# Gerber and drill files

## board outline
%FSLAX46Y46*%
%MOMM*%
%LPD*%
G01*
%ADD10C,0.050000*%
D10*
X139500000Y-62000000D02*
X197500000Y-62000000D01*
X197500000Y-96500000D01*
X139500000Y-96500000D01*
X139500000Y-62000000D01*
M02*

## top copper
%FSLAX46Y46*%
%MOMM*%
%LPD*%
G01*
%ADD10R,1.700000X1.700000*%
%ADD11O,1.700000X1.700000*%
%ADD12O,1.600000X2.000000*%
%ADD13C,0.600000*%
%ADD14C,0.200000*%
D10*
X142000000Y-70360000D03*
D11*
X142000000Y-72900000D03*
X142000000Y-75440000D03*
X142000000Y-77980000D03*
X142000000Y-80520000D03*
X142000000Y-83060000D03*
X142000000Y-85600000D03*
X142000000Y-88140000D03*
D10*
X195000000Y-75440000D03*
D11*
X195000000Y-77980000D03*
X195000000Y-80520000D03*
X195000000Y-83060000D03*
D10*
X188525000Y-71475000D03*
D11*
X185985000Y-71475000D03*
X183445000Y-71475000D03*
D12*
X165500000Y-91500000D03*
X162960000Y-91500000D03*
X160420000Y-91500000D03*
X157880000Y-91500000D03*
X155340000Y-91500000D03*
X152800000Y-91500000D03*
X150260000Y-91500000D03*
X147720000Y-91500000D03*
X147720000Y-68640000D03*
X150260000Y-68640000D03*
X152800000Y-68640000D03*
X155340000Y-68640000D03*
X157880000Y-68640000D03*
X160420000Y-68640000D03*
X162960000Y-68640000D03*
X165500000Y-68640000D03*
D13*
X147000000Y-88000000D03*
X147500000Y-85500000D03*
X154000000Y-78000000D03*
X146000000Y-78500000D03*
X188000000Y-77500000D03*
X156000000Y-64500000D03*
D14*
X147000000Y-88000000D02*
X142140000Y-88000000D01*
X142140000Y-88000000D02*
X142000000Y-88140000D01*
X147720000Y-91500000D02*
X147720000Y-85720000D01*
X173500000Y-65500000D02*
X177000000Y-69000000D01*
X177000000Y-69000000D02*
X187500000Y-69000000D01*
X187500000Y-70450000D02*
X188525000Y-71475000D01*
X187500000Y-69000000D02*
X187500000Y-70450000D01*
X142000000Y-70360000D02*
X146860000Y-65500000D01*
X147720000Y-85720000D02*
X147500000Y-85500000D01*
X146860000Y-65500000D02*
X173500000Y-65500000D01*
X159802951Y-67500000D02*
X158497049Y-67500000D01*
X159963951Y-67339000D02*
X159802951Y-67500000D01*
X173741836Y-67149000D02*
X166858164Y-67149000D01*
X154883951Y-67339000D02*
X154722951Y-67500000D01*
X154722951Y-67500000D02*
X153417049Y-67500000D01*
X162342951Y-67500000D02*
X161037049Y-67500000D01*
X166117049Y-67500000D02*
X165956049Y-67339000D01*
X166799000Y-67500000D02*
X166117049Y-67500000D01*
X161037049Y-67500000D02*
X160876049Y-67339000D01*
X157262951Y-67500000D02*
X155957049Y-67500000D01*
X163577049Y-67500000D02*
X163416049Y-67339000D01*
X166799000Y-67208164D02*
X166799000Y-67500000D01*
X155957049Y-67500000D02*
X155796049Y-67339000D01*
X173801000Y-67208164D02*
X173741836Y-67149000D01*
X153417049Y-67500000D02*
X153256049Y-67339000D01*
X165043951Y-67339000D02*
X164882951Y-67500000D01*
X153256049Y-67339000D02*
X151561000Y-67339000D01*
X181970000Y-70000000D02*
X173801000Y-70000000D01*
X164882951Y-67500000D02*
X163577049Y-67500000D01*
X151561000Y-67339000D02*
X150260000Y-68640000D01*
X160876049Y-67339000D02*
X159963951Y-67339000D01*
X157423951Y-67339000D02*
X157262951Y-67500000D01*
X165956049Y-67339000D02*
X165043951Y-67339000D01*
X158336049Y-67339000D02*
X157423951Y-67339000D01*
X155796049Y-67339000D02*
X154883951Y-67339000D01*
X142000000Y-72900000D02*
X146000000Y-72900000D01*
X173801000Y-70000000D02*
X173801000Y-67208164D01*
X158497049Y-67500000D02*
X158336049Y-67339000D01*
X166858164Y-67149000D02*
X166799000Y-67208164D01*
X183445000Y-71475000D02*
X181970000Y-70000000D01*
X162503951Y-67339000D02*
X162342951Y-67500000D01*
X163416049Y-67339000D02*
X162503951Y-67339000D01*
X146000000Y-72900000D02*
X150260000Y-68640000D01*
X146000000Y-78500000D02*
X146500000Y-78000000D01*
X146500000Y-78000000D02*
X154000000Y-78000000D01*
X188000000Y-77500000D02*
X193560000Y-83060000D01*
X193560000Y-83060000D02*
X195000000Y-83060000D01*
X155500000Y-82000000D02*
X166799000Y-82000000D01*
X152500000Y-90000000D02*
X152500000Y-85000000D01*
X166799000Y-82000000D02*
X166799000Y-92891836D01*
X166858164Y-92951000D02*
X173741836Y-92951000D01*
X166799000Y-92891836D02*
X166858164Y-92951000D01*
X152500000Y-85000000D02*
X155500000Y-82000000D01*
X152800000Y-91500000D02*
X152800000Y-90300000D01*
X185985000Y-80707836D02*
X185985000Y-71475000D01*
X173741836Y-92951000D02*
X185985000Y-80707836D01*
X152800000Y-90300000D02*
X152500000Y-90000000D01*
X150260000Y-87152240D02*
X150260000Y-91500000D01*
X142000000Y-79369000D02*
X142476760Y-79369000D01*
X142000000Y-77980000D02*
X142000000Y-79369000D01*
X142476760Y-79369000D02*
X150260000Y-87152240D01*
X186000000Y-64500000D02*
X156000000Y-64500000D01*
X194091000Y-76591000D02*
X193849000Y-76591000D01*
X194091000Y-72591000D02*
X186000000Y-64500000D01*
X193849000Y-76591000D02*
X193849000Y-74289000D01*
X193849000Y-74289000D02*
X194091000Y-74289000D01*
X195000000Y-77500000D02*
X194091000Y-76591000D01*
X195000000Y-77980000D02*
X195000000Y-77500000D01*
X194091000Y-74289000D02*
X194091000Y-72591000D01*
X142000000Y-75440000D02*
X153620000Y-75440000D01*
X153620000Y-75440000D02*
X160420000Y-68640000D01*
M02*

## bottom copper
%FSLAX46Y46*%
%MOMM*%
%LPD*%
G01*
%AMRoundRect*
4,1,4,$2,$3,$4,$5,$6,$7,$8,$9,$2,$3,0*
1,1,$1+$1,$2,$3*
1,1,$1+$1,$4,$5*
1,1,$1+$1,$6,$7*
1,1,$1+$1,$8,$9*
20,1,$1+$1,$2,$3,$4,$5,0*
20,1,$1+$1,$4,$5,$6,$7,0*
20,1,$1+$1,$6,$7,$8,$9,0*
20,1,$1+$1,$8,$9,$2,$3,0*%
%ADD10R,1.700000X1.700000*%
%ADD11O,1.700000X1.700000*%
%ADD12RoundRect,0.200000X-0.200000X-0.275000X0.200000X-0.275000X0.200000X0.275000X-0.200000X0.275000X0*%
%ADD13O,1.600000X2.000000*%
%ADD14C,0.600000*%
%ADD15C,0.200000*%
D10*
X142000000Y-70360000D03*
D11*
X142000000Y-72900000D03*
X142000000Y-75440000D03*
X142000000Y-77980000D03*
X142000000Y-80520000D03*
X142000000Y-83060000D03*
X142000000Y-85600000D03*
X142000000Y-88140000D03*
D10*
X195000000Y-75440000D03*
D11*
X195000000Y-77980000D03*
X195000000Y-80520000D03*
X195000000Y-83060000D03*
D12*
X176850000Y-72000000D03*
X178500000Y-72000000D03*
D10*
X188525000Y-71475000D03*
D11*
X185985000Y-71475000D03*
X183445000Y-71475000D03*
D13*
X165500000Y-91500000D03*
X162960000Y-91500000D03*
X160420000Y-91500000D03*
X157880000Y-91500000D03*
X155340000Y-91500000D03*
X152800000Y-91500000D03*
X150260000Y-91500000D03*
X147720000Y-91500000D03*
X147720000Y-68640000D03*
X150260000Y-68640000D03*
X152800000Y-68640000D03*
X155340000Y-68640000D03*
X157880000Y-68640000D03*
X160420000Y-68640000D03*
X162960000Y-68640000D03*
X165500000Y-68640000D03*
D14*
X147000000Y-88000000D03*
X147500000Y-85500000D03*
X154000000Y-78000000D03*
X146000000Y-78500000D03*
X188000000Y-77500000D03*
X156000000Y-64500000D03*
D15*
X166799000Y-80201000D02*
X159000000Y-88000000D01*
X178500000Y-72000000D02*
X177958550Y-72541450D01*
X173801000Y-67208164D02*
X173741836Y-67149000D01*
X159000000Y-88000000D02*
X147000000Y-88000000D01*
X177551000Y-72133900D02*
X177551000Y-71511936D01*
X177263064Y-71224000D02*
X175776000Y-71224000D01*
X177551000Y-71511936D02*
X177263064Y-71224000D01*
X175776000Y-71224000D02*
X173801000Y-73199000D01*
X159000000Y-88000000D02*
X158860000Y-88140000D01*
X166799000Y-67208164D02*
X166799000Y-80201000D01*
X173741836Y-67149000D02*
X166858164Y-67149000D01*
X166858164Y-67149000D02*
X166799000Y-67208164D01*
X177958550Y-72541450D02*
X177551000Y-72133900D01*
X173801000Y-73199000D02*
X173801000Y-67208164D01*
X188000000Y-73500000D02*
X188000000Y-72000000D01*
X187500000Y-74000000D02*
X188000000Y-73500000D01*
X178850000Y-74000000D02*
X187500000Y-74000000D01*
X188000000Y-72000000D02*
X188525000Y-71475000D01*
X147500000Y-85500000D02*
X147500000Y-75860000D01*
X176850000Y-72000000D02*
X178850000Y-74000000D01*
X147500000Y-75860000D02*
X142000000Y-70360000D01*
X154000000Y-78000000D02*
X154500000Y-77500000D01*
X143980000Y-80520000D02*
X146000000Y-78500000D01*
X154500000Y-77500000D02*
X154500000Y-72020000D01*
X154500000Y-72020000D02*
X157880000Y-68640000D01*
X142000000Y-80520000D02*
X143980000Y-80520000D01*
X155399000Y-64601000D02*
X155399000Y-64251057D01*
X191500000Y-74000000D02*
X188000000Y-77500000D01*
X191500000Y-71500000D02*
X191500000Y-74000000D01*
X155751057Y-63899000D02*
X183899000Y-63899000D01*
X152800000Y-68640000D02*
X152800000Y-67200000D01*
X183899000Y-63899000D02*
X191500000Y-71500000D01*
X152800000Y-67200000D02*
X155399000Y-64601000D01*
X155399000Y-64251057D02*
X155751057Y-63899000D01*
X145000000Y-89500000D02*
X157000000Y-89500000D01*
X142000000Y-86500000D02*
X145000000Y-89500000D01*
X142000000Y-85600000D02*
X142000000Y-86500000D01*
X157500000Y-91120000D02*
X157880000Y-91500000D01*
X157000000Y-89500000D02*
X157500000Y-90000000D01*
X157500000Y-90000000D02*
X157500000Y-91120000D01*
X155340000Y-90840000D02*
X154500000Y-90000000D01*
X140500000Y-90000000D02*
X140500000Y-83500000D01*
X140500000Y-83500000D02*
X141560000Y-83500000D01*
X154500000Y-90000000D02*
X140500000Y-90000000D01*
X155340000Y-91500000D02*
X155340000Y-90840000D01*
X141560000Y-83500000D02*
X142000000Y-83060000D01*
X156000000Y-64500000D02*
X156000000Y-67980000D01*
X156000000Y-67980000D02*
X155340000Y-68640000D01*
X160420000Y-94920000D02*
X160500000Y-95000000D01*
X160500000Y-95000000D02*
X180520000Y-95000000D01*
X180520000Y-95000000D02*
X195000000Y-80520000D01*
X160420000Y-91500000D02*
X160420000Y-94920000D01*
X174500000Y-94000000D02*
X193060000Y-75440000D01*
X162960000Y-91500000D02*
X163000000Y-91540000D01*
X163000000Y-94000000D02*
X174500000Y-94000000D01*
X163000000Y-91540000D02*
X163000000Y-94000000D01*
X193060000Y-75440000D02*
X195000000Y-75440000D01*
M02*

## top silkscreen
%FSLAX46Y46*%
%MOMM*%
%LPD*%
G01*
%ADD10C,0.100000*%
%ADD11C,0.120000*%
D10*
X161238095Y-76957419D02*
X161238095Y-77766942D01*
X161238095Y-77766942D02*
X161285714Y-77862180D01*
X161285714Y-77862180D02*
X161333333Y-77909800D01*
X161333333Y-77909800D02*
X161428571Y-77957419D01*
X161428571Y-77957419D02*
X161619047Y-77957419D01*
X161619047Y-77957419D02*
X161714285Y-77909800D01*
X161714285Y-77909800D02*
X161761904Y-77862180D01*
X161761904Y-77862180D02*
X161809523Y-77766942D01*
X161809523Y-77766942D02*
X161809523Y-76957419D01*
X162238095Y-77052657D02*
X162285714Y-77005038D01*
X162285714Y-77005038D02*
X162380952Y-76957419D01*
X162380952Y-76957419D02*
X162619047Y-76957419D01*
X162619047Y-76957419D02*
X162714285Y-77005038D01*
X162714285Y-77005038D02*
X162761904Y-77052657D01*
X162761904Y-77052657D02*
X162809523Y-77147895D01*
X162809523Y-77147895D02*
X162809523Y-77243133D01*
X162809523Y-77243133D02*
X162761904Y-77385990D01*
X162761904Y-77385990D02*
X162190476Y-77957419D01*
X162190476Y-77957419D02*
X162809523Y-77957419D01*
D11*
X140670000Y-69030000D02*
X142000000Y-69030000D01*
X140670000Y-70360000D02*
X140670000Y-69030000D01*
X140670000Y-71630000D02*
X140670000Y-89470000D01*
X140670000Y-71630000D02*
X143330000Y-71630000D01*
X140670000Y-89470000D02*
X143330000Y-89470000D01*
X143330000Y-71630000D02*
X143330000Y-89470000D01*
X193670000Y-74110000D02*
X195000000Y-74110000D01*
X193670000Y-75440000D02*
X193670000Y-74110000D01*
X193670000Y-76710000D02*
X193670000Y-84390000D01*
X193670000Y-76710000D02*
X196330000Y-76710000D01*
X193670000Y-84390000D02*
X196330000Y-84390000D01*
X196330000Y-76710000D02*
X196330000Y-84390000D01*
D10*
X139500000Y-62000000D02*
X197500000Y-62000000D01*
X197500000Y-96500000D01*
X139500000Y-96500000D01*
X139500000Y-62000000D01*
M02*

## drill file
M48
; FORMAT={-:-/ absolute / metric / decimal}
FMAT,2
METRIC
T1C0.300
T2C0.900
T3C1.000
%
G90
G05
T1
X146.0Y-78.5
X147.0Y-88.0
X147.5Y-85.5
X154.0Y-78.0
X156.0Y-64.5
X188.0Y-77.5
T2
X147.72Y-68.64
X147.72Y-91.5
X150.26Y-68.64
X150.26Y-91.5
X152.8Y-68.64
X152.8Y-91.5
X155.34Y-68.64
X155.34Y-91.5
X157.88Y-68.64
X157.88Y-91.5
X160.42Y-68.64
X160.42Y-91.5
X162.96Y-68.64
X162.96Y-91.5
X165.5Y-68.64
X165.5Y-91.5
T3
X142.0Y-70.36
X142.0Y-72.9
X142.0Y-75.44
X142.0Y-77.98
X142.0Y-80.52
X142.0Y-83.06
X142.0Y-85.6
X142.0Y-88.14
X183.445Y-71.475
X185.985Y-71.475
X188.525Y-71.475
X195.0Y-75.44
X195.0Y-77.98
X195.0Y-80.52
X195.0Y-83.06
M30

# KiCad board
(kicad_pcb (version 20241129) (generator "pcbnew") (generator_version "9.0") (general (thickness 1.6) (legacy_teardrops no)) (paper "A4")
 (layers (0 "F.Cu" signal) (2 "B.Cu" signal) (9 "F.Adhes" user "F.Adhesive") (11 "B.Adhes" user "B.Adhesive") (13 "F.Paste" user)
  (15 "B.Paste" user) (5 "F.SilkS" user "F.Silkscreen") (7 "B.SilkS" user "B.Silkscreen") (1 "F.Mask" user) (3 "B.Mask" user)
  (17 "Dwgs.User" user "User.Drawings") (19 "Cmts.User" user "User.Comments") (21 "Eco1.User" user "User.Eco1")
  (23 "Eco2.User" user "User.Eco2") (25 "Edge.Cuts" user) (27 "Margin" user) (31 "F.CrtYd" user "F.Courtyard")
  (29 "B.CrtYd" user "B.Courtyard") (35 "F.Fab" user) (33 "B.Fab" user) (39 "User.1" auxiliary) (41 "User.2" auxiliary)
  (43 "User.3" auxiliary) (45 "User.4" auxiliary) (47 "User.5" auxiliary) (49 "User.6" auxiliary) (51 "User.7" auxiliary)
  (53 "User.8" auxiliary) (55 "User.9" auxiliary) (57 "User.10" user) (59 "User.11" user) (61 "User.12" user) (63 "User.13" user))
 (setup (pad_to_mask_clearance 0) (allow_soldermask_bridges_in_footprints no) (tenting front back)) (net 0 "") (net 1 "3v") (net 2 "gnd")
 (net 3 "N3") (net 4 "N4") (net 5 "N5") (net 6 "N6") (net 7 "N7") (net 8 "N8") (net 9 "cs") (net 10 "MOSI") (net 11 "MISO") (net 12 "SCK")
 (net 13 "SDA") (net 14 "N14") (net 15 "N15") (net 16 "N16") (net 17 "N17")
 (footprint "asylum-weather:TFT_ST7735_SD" (layer "F.Cu") (at 162 79)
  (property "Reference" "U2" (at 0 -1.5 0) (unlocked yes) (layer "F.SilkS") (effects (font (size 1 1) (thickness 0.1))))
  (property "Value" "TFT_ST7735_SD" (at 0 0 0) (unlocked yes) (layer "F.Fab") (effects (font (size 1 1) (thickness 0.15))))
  (fp_line (start -21.33 -9.97) (end -20 -9.97) (stroke (width 0.12) (type solid)) (layer "F.SilkS"))
  (fp_line (start -21.33 -8.64) (end -21.33 -9.97) (stroke (width 0.12) (type solid)) (layer "F.SilkS"))
  (fp_line (start -21.33 -7.37) (end -21.33 10.47) (stroke (width 0.12) (type solid)) (layer "F.SilkS"))
  (fp_line (start -21.33 -7.37) (end -18.67 -7.37) (stroke (width 0.12) (type solid)) (layer "F.SilkS"))
  (fp_line (start -21.33 10.47) (end -18.67 10.47) (stroke (width 0.12) (type solid)) (layer "F.SilkS"))
  (fp_line (start -18.67 -7.37) (end -18.67 10.47) (stroke (width 0.12) (type solid)) (layer "F.SilkS"))
  (fp_line (start 31.67 -4.89) (end 33 -4.89) (stroke (width 0.12) (type solid)) (layer "F.SilkS"))
  (fp_line (start 31.67 -3.56) (end 31.67 -4.89) (stroke (width 0.12) (type solid)) (layer "F.SilkS"))
  (fp_line (start 31.67 -2.29) (end 31.67 5.39) (stroke (width 0.12) (type solid)) (layer "F.SilkS"))
  (fp_line (start 31.67 -2.29) (end 34.33 -2.29) (stroke (width 0.12) (type solid)) (layer "F.SilkS"))
  (fp_line (start 31.67 5.39) (end 34.33 5.39) (stroke (width 0.12) (type solid)) (layer "F.SilkS"))
  (fp_line (start 34.33 -2.29) (end 34.33 5.39) (stroke (width 0.12) (type solid)) (layer "F.SilkS"))
  (fp_rect (start -22.5 -17) (end 35.5 17.5) (stroke (width 0.1) (type default)) (fill no) (layer "F.SilkS"))
  (pad "1" thru_hole rect (at -20 -8.64) (size 1.7 1.7) (drill 1) (layers "*.Cu" "*.Mask") (remove_unused_layers no) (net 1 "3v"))
  (pad "2" thru_hole oval (at -20 -6.1) (size 1.7 1.7) (drill 1) (layers "*.Cu" "*.Mask") (remove_unused_layers no) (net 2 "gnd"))
  (pad "3" thru_hole oval (at -20 -3.56) (size 1.7 1.7) (drill 1) (layers "*.Cu" "*.Mask") (remove_unused_layers no) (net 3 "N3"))
  (pad "4" thru_hole oval (at -20 -1.02) (size 1.7 1.7) (drill 1) (layers "*.Cu" "*.Mask") (remove_unused_layers no) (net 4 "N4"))
  (pad "5" thru_hole oval (at -20 1.52) (size 1.7 1.7) (drill 1) (layers "*.Cu" "*.Mask") (remove_unused_layers no) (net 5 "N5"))
  (pad "6" thru_hole oval (at -20 4.06) (size 1.7 1.7) (drill 1) (layers "*.Cu" "*.Mask") (remove_unused_layers no) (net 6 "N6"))
  (pad "7" thru_hole oval (at -20 6.6) (size 1.7 1.7) (drill 1) (layers "*.Cu" "*.Mask") (remove_unused_layers no) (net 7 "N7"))
  (pad "8" thru_hole oval (at -20 9.14) (size 1.7 1.7) (drill 1) (layers "*.Cu" "*.Mask") (remove_unused_layers no) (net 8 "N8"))
  (pad "9" thru_hole rect (at 33 -3.56) (size 1.7 1.7) (drill 1) (layers "*.Cu" "*.Mask") (remove_unused_layers no) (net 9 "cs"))
  (pad "10" thru_hole oval (at 33 -1.02) (size 1.7 1.7) (drill 1) (layers "*.Cu" "*.Mask") (remove_unused_layers no) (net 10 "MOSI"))
  (pad "11" thru_hole oval (at 33 1.52) (size 1.7 1.7) (drill 1) (layers "*.Cu" "*.Mask") (remove_unused_layers no) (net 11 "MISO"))
  (pad "12" thru_hole oval (at 33 4.06) (size 1.7 1.7) (drill 1) (layers "*.Cu" "*.Mask") (remove_unused_layers no) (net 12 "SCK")))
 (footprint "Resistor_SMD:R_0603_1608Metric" (layer "B.Cu") (at 177.675 72)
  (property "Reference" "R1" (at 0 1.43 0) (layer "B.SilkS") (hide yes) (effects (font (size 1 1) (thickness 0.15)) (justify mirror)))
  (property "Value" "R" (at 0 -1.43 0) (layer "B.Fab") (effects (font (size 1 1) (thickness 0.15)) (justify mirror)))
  (pad "1" smd roundrect (at -0.825 0) (size 0.8 0.95) (layers "B.Cu" "B.Mask" "B.Paste") (roundrect_rratio 0.25) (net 1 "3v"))
  (pad "2" smd roundrect (at 0.825 0) (size 0.8 0.95) (layers "B.Cu" "B.Mask" "B.Paste") (roundrect_rratio 0.25) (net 8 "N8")))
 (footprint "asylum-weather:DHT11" (layer "B.Cu") (at 188.525 71.475 90)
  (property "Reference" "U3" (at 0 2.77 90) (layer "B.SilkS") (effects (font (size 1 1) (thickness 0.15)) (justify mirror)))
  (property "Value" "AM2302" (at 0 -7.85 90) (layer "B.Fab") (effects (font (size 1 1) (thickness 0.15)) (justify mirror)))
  (pad "1" thru_hole rect (at 0 0 90) (size 1.7 1.7) (drill 1) (layers "F&B.Cu" "*.Mask") (remove_unused_layers no) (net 1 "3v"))
  (pad "2" thru_hole oval (at 0 -2.54 90) (size 1.7 1.7) (drill 1) (layers "F&B.Cu" "*.Mask") (remove_unused_layers no) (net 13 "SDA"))
  (pad "3" thru_hole oval (at 0 -5.08 90) (size 1.7 1.7) (drill 1) (layers "F&B.Cu" "*.Mask") (remove_unused_layers no) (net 2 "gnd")))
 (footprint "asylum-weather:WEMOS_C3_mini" (layer "B.Cu") (at 158 80.07 90)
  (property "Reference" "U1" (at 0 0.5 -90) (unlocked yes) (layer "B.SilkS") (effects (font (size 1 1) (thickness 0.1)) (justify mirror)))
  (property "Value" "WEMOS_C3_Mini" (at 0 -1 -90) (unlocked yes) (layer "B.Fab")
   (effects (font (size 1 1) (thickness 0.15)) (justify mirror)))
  (pad "1" thru_hole oval (at -11.43 7.5 90) (size 2 1.6) (drill 0.9) (layers "F&B.Cu" "*.Mask") (remove_unused_layers no) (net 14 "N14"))
  (pad "2" thru_hole oval (at -11.43 4.96 90) (size 2 1.6) (drill 0.9) (layers "F&B.Cu" "*.Mask") (remove_unused_layers no) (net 9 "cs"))
  (pad "3" thru_hole oval (at -11.43 2.42 90) (size 2 1.6) (drill 0.9) (layers "F&B.Cu" "*.Mask") (remove_unused_layers no) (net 11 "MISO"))
  (pad "4" thru_hole oval (at -11.43 -0.12 90) (size 2 1.6) (drill 0.9) (layers "F&B.Cu" "*.Mask") (remove_unused_layers no) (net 7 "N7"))
  (pad "5" thru_hole oval (at -11.43 -2.66 90) (size 2 1.6) (drill 0.9) (layers "F&B.Cu" "*.Mask") (remove_unused_layers no) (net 6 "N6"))
  (pad "6" thru_hole oval (at -11.43 -5.2 90) (size 2 1.6) (drill 0.9) (layers "F&B.Cu" "*.Mask") (remove_unused_layers no) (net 13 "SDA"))
  (pad "7" thru_hole oval (at -11.43 -7.74 90) (size 2 1.6) (drill 0.9) (layers "F&B.Cu" "*.Mask") (remove_unused_layers no) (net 4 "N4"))
  (pad "8" thru_hole oval (at -11.43 -10.28 90) (size 2 1.6) (drill 0.9) (layers "F&B.Cu" "*.Mask") (remove_unused_layers no) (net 1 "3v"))
  (pad "9" thru_hole oval (at 11.43 -10.28 90) (size 2 1.6) (drill 0.9) (layers "F&B.Cu" "*.Mask") (remove_unused_layers no) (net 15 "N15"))
  (pad "10" thru_hole oval (at 11.43 -7.74 90) (size 2 1.6) (drill 0.9) (layers "F&B.Cu" "*.Mask") (remove_unused_layers no) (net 2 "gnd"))
  (pad "11" thru_hole oval (at 11.43 -5.2 90) (size 2 1.6) (drill 0.9) (layers "F&B.Cu" "*.Mask") (remove_unused_layers no) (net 12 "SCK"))
  (pad "12" thru_hole oval (at 11.43 -2.66 90) (size 2 1.6) (drill 0.9) (layers "F&B.Cu" "*.Mask") (remove_unused_layers no) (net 10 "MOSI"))
  (pad "13" thru_hole oval (at 11.43 -0.12 90) (size 2 1.6) (drill 0.9) (layers "F&B.Cu" "*.Mask") (remove_unused_layers no) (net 5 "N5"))
  (pad "14" thru_hole oval (at 11.43 2.42 90) (size 2 1.6) (drill 0.9) (layers "F&B.Cu" "*.Mask") (remove_unused_layers no) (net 3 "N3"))
  (pad "15" thru_hole oval (at 11.43 4.96 90) (size 2 1.6) (drill 0.9) (layers "F&B.Cu" "*.Mask") (remove_unused_layers no) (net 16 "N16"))
  (pad "16" thru_hole oval (at 11.43 7.5 90) (size 2 1.6) (drill 0.9) (layers "F&B.Cu" "*.Mask") (remove_unused_layers no) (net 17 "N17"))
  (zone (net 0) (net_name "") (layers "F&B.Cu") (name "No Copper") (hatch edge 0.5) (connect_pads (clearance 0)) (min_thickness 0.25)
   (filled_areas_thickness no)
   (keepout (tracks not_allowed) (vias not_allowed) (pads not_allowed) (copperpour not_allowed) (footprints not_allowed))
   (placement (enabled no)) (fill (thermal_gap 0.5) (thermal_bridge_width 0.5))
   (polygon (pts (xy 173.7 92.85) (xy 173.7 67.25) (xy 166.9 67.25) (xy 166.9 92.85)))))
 (gr_rect (start 139.5 62) (end 197.5 96.5) (stroke (width 0.05) (type default)) (fill no) (layer "Edge.Cuts"))
 (segment (start 147 88) (end 142.14 88) (width 0.2) (layer "F.Cu") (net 8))
 (segment (start 142.14 88) (end 142 88.14) (width 0.2) (layer "F.Cu") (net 8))
 (via (at 147 88) (size 0.6) (drill 0.3) (layers "F.Cu" "B.Cu") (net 8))
 (segment (start 166.799 80.201) (end 159 88) (width 0.2) (layer "B.Cu") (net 8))
 (segment (start 178.5 72) (end 177.95855 72.54145) (width 0.2) (layer "B.Cu") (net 8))
 (segment (start 173.801 67.208164) (end 173.741836 67.149) (width 0.2) (layer "B.Cu") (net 8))
 (segment (start 159 88) (end 147 88) (width 0.2) (layer "B.Cu") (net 8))
 (segment (start 177.551 72.1339) (end 177.551 71.511936) (width 0.2) (layer "B.Cu") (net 8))
 (segment (start 177.263064 71.224) (end 175.776 71.224) (width 0.2) (layer "B.Cu") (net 8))
 (segment (start 177.551 71.511936) (end 177.263064 71.224) (width 0.2) (layer "B.Cu") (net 8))
 (segment (start 175.776 71.224) (end 173.801 73.199) (width 0.2) (layer "B.Cu") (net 8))
 (segment (start 159 88) (end 158.86 88.14) (width 0.2) (layer "B.Cu") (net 8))
 (segment (start 166.799 67.208164) (end 166.799 80.201) (width 0.2) (layer "B.Cu") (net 8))
 (segment (start 173.741836 67.149) (end 166.858164 67.149) (width 0.2) (layer "B.Cu") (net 8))
 (segment (start 166.858164 67.149) (end 166.799 67.208164) (width 0.2) (layer "B.Cu") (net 8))
 (segment (start 177.95855 72.54145) (end 177.551 72.1339) (width 0.2) (layer "B.Cu") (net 8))
 (segment (start 173.801 73.199) (end 173.801 67.208164) (width 0.2) (layer "B.Cu") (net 8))
 (segment (start 147.72 91.5) (end 147.72 85.72) (width 0.2) (layer "F.Cu") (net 1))
 (segment (start 173.5 65.5) (end 177 69) (width 0.2) (layer "F.Cu") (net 1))
 (segment (start 177 69) (end 187.5 69) (width 0.2) (layer "F.Cu") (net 1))
 (segment (start 187.5 70.45) (end 188.525 71.475) (width 0.2) (layer "F.Cu") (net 1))
 (segment (start 187.5 69) (end 187.5 70.45) (width 0.2) (layer "F.Cu") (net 1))
 (segment (start 142 70.36) (end 146.86 65.5) (width 0.2) (layer "F.Cu") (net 1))
 (segment (start 147.72 85.72) (end 147.5 85.5) (width 0.2) (layer "F.Cu") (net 1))
 (segment (start 146.86 65.5) (end 173.5 65.5) (width 0.2) (layer "F.Cu") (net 1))
 (via (at 147.5 85.5) (size 0.6) (drill 0.3) (layers "F.Cu" "B.Cu") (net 1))
 (segment (start 188 73.5) (end 188 72) (width 0.2) (layer "B.Cu") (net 1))
 (segment (start 187.5 74) (end 188 73.5) (width 0.2) (layer "B.Cu") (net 1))
 (segment (start 178.85 74) (end 187.5 74) (width 0.2) (layer "B.Cu") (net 1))
 (segment (start 188 72) (end 188.525 71.475) (width 0.2) (layer "B.Cu") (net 1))
 (segment (start 147.5 85.5) (end 147.5 75.86) (width 0.2) (layer "B.Cu") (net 1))
 (segment (start 176.85 72) (end 178.85 74) (width 0.2) (layer "B.Cu") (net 1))
 (segment (start 147.5 75.86) (end 142 70.36) (width 0.2) (layer "B.Cu") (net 1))
 (segment (start 159.802951 67.5) (end 158.497049 67.5) (width 0.2) (layer "F.Cu") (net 2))
 (segment (start 159.963951 67.339) (end 159.802951 67.5) (width 0.2) (layer "F.Cu") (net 2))
 (segment (start 173.741836 67.149) (end 166.858164 67.149) (width 0.2) (layer "F.Cu") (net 2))
 (segment (start 154.883951 67.339) (end 154.722951 67.5) (width 0.2) (layer "F.Cu") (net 2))
 (segment (start 154.722951 67.5) (end 153.417049 67.5) (width 0.2) (layer "F.Cu") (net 2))
 (segment (start 162.342951 67.5) (end 161.037049 67.5) (width 0.2) (layer "F.Cu") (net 2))
 (segment (start 166.117049 67.5) (end 165.956049 67.339) (width 0.2) (layer "F.Cu") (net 2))
 (segment (start 166.799 67.5) (end 166.117049 67.5) (width 0.2) (layer "F.Cu") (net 2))
 (segment (start 161.037049 67.5) (end 160.876049 67.339) (width 0.2) (layer "F.Cu") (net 2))
 (segment (start 157.262951 67.5) (end 155.957049 67.5) (width 0.2) (layer "F.Cu") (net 2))
 (segment (start 163.577049 67.5) (end 163.416049 67.339) (width 0.2) (layer "F.Cu") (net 2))
 (segment (start 166.799 67.208164) (end 166.799 67.5) (width 0.2) (layer "F.Cu") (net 2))
 (segment (start 155.957049 67.5) (end 155.796049 67.339) (width 0.2) (layer "F.Cu") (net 2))
 (segment (start 173.801 67.208164) (end 173.741836 67.149) (width 0.2) (layer "F.Cu") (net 2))
 (segment (start 153.417049 67.5) (end 153.256049 67.339) (width 0.2) (layer "F.Cu") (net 2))
 (segment (start 165.043951 67.339) (end 164.882951 67.5) (width 0.2) (layer "F.Cu") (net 2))
 (segment (start 153.256049 67.339) (end 151.561 67.339) (width 0.2) (layer "F.Cu") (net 2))
 (segment (start 181.97 70) (end 173.801 70) (width 0.2) (layer "F.Cu") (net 2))
 (segment (start 164.882951 67.5) (end 163.577049 67.5) (width 0.2) (layer "F.Cu") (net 2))
 (segment (start 151.561 67.339) (end 150.26 68.64) (width 0.2) (layer "F.Cu") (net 2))
 (segment (start 160.876049 67.339) (end 159.963951 67.339) (width 0.2) (layer "F.Cu") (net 2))
 (segment (start 157.423951 67.339) (end 157.262951 67.5) (width 0.2) (layer "F.Cu") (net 2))
 (segment (start 165.956049 67.339) (end 165.043951 67.339) (width 0.2) (layer "F.Cu") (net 2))
 (segment (start 158.336049 67.339) (end 157.423951 67.339) (width 0.2) (layer "F.Cu") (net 2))
 (segment (start 155.796049 67.339) (end 154.883951 67.339) (width 0.2) (layer "F.Cu") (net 2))
 (segment (start 142 72.9) (end 146 72.9) (width 0.2) (layer "F.Cu") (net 2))
 (segment (start 173.801 70) (end 173.801 67.208164) (width 0.2) (layer "F.Cu") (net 2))
 (segment (start 158.497049 67.5) (end 158.336049 67.339) (width 0.2) (layer "F.Cu") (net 2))
 (segment (start 166.858164 67.149) (end 166.799 67.208164) (width 0.2) (layer "F.Cu") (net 2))
 (segment (start 183.445 71.475) (end 181.97 70) (width 0.2) (layer "F.Cu") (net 2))
 (segment (start 162.503951 67.339) (end 162.342951 67.5) (width 0.2) (layer "F.Cu") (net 2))
 (segment (start 163.416049 67.339) (end 162.503951 67.339) (width 0.2) (layer "F.Cu") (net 2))
 (segment (start 146 72.9) (end 150.26 68.64) (width 0.2) (layer "F.Cu") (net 2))
 (segment (start 146 78.5) (end 146.5 78) (width 0.2) (layer "F.Cu") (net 5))
 (segment (start 146.5 78) (end 154 78) (width 0.2) (layer "F.Cu") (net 5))
 (via (at 154 78) (size 0.6) (drill 0.3) (layers "F.Cu" "B.Cu") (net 5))
 (via (at 146 78.5) (size 0.6) (drill 0.3) (layers "F.Cu" "B.Cu") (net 5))
 (segment (start 154 78) (end 154.5 77.5) (width 0.2) (layer "B.Cu") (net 5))
 (segment (start 143.98 80.52) (end 146 78.5) (width 0.2) (layer "B.Cu") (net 5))
 (segment (start 154.5 77.5) (end 154.5 72.02) (width 0.2) (layer "B.Cu") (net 5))
 (segment (start 154.5 72.02) (end 157.88 68.64) (width 0.2) (layer "B.Cu") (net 5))
 (segment (start 142 80.52) (end 143.98 80.52) (width 0.2) (layer "B.Cu") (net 5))
 (segment (start 188 77.5) (end 193.56 83.06) (width 0.2) (layer "F.Cu") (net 12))
 (segment (start 193.56 83.06) (end 195 83.06) (width 0.2) (layer "F.Cu") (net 12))
 (via (at 188 77.5) (size 0.6) (drill 0.3) (layers "F.Cu" "B.Cu") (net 12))
 (segment (start 155.399 64.601) (end 155.399 64.251057) (width 0.2) (layer "B.Cu") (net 12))
 (segment (start 191.5 74) (end 188 77.5) (width 0.2) (layer "B.Cu") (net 12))
 (segment (start 191.5 71.5) (end 191.5 74) (width 0.2) (layer "B.Cu") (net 12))
 (segment (start 155.751057 63.899) (end 183.899 63.899) (width 0.2) (layer "B.Cu") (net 12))
 (segment (start 152.8 68.64) (end 152.8 67.2) (width 0.2) (layer "B.Cu") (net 12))
 (segment (start 183.899 63.899) (end 191.5 71.5) (width 0.2) (layer "B.Cu") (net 12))
 (segment (start 152.8 67.2) (end 155.399 64.601) (width 0.2) (layer "B.Cu") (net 12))
 (segment (start 155.399 64.251057) (end 155.751057 63.899) (width 0.2) (layer "B.Cu") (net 12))
 (segment (start 155.5 82) (end 166.799 82) (width 0.2) (layer "F.Cu") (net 13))
 (segment (start 152.5 90) (end 152.5 85) (width 0.2) (layer "F.Cu") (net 13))
 (segment (start 166.799 82) (end 166.799 92.891836) (width 0.2) (layer "F.Cu") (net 13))
 (segment (start 166.858164 92.951) (end 173.741836 92.951) (width 0.2) (layer "F.Cu") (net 13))
 (segment (start 166.799 92.891836) (end 166.858164 92.951) (width 0.2) (layer "F.Cu") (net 13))
 (segment (start 152.5 85) (end 155.5 82) (width 0.2) (layer "F.Cu") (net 13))
 (segment (start 152.8 91.5) (end 152.8 90.3) (width 0.2) (layer "F.Cu") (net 13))
 (segment (start 185.985 80.707836) (end 185.985 71.475) (width 0.2) (layer "F.Cu") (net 13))
 (segment (start 173.741836 92.951) (end 185.985 80.707836) (width 0.2) (layer "F.Cu") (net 13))
 (segment (start 152.8 90.3) (end 152.5 90) (width 0.2) (layer "F.Cu") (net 13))
 (segment (start 145 89.5) (end 157 89.5) (width 0.2) (layer "B.Cu") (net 7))
 (segment (start 142 86.5) (end 145 89.5) (width 0.2) (layer "B.Cu") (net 7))
 (segment (start 142 85.6) (end 142 86.5) (width 0.2) (layer "B.Cu") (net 7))
 (segment (start 157.5 91.12) (end 157.88 91.5) (width 0.2) (layer "B.Cu") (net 7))
 (segment (start 157 89.5) (end 157.5 90) (width 0.2) (layer "B.Cu") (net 7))
 (segment (start 157.5 90) (end 157.5 91.12) (width 0.2) (layer "B.Cu") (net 7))
 (segment (start 150.26 87.15224) (end 150.26 91.5) (width 0.2) (layer "F.Cu") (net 4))
 (segment (start 142 79.369) (end 142.47676 79.369) (width 0.2) (layer "F.Cu") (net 4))
 (segment (start 142 77.98) (end 142 79.369) (width 0.2) (layer "F.Cu") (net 4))
 (segment (start 142.47676 79.369) (end 150.26 87.15224) (width 0.2) (layer "F.Cu") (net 4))
 (segment (start 155.34 90.84) (end 154.5 90) (width 0.2) (layer "B.Cu") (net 6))
 (segment (start 140.5 90) (end 140.5 83.5) (width 0.2) (layer "B.Cu") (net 6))
 (segment (start 140.5 83.5) (end 141.56 83.5) (width 0.2) (layer "B.Cu") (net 6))
 (segment (start 154.5 90) (end 140.5 90) (width 0.2) (layer "B.Cu") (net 6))
 (segment (start 155.34 91.5) (end 155.34 90.84) (width 0.2) (layer "B.Cu") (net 6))
 (segment (start 141.56 83.5) (end 142 83.06) (width 0.2) (layer "B.Cu") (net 6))
 (segment (start 186 64.5) (end 156 64.5) (width 0.2) (layer "F.Cu") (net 10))
 (segment (start 194.091 76.591) (end 193.849 76.591) (width 0.2) (layer "F.Cu") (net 10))
 (segment (start 194.091 72.591) (end 186 64.5) (width 0.2) (layer "F.Cu") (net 10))
 (segment (start 193.849 76.591) (end 193.849 74.289) (width 0.2) (layer "F.Cu") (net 10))
 (segment (start 193.849 74.289) (end 194.091 74.289) (width 0.2) (layer "F.Cu") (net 10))
 (segment (start 195 77.5) (end 194.091 76.591) (width 0.2) (layer "F.Cu") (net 10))
 (segment (start 195 77.98) (end 195 77.5) (width 0.2) (layer "F.Cu") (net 10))
 (segment (start 194.091 74.289) (end 194.091 72.591) (width 0.2) (layer "F.Cu") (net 10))
 (via (at 156 64.5) (size 0.6) (drill 0.3) (layers "F.Cu" "B.Cu") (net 10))
 (segment (start 156 64.5) (end 156 67.98) (width 0.2) (layer "B.Cu") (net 10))
 (segment (start 156 67.98) (end 155.34 68.64) (width 0.2) (layer "B.Cu") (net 10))
 (segment (start 142 75.44) (end 153.62 75.44) (width 0.2) (layer "F.Cu") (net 3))
 (segment (start 153.62 75.44) (end 160.42 68.64) (width 0.2) (layer "F.Cu") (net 3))
 (segment (start 160.42 94.92) (end 160.5 95) (width 0.2) (layer "B.Cu") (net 11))
 (segment (start 160.5 95) (end 180.52 95) (width 0.2) (layer "B.Cu") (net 11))
 (segment (start 180.52 95) (end 195 80.52) (width 0.2) (layer "B.Cu") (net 11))
 (segment (start 160.42 91.5) (end 160.42 94.92) (width 0.2) (layer "B.Cu") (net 11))
 (segment (start 174.5 94) (end 193.06 75.44) (width 0.2) (layer "B.Cu") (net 9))
 (segment (start 162.96 91.5) (end 163 91.54) (width 0.2) (layer "B.Cu") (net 9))
 (segment (start 163 94) (end 174.5 94) (width 0.2) (layer "B.Cu") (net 9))
 (segment (start 163 91.54) (end 163 94) (width 0.2) (layer "B.Cu") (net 9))
 (segment (start 193.06 75.44) (end 195 75.44) (width 0.2) (layer "B.Cu") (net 9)))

